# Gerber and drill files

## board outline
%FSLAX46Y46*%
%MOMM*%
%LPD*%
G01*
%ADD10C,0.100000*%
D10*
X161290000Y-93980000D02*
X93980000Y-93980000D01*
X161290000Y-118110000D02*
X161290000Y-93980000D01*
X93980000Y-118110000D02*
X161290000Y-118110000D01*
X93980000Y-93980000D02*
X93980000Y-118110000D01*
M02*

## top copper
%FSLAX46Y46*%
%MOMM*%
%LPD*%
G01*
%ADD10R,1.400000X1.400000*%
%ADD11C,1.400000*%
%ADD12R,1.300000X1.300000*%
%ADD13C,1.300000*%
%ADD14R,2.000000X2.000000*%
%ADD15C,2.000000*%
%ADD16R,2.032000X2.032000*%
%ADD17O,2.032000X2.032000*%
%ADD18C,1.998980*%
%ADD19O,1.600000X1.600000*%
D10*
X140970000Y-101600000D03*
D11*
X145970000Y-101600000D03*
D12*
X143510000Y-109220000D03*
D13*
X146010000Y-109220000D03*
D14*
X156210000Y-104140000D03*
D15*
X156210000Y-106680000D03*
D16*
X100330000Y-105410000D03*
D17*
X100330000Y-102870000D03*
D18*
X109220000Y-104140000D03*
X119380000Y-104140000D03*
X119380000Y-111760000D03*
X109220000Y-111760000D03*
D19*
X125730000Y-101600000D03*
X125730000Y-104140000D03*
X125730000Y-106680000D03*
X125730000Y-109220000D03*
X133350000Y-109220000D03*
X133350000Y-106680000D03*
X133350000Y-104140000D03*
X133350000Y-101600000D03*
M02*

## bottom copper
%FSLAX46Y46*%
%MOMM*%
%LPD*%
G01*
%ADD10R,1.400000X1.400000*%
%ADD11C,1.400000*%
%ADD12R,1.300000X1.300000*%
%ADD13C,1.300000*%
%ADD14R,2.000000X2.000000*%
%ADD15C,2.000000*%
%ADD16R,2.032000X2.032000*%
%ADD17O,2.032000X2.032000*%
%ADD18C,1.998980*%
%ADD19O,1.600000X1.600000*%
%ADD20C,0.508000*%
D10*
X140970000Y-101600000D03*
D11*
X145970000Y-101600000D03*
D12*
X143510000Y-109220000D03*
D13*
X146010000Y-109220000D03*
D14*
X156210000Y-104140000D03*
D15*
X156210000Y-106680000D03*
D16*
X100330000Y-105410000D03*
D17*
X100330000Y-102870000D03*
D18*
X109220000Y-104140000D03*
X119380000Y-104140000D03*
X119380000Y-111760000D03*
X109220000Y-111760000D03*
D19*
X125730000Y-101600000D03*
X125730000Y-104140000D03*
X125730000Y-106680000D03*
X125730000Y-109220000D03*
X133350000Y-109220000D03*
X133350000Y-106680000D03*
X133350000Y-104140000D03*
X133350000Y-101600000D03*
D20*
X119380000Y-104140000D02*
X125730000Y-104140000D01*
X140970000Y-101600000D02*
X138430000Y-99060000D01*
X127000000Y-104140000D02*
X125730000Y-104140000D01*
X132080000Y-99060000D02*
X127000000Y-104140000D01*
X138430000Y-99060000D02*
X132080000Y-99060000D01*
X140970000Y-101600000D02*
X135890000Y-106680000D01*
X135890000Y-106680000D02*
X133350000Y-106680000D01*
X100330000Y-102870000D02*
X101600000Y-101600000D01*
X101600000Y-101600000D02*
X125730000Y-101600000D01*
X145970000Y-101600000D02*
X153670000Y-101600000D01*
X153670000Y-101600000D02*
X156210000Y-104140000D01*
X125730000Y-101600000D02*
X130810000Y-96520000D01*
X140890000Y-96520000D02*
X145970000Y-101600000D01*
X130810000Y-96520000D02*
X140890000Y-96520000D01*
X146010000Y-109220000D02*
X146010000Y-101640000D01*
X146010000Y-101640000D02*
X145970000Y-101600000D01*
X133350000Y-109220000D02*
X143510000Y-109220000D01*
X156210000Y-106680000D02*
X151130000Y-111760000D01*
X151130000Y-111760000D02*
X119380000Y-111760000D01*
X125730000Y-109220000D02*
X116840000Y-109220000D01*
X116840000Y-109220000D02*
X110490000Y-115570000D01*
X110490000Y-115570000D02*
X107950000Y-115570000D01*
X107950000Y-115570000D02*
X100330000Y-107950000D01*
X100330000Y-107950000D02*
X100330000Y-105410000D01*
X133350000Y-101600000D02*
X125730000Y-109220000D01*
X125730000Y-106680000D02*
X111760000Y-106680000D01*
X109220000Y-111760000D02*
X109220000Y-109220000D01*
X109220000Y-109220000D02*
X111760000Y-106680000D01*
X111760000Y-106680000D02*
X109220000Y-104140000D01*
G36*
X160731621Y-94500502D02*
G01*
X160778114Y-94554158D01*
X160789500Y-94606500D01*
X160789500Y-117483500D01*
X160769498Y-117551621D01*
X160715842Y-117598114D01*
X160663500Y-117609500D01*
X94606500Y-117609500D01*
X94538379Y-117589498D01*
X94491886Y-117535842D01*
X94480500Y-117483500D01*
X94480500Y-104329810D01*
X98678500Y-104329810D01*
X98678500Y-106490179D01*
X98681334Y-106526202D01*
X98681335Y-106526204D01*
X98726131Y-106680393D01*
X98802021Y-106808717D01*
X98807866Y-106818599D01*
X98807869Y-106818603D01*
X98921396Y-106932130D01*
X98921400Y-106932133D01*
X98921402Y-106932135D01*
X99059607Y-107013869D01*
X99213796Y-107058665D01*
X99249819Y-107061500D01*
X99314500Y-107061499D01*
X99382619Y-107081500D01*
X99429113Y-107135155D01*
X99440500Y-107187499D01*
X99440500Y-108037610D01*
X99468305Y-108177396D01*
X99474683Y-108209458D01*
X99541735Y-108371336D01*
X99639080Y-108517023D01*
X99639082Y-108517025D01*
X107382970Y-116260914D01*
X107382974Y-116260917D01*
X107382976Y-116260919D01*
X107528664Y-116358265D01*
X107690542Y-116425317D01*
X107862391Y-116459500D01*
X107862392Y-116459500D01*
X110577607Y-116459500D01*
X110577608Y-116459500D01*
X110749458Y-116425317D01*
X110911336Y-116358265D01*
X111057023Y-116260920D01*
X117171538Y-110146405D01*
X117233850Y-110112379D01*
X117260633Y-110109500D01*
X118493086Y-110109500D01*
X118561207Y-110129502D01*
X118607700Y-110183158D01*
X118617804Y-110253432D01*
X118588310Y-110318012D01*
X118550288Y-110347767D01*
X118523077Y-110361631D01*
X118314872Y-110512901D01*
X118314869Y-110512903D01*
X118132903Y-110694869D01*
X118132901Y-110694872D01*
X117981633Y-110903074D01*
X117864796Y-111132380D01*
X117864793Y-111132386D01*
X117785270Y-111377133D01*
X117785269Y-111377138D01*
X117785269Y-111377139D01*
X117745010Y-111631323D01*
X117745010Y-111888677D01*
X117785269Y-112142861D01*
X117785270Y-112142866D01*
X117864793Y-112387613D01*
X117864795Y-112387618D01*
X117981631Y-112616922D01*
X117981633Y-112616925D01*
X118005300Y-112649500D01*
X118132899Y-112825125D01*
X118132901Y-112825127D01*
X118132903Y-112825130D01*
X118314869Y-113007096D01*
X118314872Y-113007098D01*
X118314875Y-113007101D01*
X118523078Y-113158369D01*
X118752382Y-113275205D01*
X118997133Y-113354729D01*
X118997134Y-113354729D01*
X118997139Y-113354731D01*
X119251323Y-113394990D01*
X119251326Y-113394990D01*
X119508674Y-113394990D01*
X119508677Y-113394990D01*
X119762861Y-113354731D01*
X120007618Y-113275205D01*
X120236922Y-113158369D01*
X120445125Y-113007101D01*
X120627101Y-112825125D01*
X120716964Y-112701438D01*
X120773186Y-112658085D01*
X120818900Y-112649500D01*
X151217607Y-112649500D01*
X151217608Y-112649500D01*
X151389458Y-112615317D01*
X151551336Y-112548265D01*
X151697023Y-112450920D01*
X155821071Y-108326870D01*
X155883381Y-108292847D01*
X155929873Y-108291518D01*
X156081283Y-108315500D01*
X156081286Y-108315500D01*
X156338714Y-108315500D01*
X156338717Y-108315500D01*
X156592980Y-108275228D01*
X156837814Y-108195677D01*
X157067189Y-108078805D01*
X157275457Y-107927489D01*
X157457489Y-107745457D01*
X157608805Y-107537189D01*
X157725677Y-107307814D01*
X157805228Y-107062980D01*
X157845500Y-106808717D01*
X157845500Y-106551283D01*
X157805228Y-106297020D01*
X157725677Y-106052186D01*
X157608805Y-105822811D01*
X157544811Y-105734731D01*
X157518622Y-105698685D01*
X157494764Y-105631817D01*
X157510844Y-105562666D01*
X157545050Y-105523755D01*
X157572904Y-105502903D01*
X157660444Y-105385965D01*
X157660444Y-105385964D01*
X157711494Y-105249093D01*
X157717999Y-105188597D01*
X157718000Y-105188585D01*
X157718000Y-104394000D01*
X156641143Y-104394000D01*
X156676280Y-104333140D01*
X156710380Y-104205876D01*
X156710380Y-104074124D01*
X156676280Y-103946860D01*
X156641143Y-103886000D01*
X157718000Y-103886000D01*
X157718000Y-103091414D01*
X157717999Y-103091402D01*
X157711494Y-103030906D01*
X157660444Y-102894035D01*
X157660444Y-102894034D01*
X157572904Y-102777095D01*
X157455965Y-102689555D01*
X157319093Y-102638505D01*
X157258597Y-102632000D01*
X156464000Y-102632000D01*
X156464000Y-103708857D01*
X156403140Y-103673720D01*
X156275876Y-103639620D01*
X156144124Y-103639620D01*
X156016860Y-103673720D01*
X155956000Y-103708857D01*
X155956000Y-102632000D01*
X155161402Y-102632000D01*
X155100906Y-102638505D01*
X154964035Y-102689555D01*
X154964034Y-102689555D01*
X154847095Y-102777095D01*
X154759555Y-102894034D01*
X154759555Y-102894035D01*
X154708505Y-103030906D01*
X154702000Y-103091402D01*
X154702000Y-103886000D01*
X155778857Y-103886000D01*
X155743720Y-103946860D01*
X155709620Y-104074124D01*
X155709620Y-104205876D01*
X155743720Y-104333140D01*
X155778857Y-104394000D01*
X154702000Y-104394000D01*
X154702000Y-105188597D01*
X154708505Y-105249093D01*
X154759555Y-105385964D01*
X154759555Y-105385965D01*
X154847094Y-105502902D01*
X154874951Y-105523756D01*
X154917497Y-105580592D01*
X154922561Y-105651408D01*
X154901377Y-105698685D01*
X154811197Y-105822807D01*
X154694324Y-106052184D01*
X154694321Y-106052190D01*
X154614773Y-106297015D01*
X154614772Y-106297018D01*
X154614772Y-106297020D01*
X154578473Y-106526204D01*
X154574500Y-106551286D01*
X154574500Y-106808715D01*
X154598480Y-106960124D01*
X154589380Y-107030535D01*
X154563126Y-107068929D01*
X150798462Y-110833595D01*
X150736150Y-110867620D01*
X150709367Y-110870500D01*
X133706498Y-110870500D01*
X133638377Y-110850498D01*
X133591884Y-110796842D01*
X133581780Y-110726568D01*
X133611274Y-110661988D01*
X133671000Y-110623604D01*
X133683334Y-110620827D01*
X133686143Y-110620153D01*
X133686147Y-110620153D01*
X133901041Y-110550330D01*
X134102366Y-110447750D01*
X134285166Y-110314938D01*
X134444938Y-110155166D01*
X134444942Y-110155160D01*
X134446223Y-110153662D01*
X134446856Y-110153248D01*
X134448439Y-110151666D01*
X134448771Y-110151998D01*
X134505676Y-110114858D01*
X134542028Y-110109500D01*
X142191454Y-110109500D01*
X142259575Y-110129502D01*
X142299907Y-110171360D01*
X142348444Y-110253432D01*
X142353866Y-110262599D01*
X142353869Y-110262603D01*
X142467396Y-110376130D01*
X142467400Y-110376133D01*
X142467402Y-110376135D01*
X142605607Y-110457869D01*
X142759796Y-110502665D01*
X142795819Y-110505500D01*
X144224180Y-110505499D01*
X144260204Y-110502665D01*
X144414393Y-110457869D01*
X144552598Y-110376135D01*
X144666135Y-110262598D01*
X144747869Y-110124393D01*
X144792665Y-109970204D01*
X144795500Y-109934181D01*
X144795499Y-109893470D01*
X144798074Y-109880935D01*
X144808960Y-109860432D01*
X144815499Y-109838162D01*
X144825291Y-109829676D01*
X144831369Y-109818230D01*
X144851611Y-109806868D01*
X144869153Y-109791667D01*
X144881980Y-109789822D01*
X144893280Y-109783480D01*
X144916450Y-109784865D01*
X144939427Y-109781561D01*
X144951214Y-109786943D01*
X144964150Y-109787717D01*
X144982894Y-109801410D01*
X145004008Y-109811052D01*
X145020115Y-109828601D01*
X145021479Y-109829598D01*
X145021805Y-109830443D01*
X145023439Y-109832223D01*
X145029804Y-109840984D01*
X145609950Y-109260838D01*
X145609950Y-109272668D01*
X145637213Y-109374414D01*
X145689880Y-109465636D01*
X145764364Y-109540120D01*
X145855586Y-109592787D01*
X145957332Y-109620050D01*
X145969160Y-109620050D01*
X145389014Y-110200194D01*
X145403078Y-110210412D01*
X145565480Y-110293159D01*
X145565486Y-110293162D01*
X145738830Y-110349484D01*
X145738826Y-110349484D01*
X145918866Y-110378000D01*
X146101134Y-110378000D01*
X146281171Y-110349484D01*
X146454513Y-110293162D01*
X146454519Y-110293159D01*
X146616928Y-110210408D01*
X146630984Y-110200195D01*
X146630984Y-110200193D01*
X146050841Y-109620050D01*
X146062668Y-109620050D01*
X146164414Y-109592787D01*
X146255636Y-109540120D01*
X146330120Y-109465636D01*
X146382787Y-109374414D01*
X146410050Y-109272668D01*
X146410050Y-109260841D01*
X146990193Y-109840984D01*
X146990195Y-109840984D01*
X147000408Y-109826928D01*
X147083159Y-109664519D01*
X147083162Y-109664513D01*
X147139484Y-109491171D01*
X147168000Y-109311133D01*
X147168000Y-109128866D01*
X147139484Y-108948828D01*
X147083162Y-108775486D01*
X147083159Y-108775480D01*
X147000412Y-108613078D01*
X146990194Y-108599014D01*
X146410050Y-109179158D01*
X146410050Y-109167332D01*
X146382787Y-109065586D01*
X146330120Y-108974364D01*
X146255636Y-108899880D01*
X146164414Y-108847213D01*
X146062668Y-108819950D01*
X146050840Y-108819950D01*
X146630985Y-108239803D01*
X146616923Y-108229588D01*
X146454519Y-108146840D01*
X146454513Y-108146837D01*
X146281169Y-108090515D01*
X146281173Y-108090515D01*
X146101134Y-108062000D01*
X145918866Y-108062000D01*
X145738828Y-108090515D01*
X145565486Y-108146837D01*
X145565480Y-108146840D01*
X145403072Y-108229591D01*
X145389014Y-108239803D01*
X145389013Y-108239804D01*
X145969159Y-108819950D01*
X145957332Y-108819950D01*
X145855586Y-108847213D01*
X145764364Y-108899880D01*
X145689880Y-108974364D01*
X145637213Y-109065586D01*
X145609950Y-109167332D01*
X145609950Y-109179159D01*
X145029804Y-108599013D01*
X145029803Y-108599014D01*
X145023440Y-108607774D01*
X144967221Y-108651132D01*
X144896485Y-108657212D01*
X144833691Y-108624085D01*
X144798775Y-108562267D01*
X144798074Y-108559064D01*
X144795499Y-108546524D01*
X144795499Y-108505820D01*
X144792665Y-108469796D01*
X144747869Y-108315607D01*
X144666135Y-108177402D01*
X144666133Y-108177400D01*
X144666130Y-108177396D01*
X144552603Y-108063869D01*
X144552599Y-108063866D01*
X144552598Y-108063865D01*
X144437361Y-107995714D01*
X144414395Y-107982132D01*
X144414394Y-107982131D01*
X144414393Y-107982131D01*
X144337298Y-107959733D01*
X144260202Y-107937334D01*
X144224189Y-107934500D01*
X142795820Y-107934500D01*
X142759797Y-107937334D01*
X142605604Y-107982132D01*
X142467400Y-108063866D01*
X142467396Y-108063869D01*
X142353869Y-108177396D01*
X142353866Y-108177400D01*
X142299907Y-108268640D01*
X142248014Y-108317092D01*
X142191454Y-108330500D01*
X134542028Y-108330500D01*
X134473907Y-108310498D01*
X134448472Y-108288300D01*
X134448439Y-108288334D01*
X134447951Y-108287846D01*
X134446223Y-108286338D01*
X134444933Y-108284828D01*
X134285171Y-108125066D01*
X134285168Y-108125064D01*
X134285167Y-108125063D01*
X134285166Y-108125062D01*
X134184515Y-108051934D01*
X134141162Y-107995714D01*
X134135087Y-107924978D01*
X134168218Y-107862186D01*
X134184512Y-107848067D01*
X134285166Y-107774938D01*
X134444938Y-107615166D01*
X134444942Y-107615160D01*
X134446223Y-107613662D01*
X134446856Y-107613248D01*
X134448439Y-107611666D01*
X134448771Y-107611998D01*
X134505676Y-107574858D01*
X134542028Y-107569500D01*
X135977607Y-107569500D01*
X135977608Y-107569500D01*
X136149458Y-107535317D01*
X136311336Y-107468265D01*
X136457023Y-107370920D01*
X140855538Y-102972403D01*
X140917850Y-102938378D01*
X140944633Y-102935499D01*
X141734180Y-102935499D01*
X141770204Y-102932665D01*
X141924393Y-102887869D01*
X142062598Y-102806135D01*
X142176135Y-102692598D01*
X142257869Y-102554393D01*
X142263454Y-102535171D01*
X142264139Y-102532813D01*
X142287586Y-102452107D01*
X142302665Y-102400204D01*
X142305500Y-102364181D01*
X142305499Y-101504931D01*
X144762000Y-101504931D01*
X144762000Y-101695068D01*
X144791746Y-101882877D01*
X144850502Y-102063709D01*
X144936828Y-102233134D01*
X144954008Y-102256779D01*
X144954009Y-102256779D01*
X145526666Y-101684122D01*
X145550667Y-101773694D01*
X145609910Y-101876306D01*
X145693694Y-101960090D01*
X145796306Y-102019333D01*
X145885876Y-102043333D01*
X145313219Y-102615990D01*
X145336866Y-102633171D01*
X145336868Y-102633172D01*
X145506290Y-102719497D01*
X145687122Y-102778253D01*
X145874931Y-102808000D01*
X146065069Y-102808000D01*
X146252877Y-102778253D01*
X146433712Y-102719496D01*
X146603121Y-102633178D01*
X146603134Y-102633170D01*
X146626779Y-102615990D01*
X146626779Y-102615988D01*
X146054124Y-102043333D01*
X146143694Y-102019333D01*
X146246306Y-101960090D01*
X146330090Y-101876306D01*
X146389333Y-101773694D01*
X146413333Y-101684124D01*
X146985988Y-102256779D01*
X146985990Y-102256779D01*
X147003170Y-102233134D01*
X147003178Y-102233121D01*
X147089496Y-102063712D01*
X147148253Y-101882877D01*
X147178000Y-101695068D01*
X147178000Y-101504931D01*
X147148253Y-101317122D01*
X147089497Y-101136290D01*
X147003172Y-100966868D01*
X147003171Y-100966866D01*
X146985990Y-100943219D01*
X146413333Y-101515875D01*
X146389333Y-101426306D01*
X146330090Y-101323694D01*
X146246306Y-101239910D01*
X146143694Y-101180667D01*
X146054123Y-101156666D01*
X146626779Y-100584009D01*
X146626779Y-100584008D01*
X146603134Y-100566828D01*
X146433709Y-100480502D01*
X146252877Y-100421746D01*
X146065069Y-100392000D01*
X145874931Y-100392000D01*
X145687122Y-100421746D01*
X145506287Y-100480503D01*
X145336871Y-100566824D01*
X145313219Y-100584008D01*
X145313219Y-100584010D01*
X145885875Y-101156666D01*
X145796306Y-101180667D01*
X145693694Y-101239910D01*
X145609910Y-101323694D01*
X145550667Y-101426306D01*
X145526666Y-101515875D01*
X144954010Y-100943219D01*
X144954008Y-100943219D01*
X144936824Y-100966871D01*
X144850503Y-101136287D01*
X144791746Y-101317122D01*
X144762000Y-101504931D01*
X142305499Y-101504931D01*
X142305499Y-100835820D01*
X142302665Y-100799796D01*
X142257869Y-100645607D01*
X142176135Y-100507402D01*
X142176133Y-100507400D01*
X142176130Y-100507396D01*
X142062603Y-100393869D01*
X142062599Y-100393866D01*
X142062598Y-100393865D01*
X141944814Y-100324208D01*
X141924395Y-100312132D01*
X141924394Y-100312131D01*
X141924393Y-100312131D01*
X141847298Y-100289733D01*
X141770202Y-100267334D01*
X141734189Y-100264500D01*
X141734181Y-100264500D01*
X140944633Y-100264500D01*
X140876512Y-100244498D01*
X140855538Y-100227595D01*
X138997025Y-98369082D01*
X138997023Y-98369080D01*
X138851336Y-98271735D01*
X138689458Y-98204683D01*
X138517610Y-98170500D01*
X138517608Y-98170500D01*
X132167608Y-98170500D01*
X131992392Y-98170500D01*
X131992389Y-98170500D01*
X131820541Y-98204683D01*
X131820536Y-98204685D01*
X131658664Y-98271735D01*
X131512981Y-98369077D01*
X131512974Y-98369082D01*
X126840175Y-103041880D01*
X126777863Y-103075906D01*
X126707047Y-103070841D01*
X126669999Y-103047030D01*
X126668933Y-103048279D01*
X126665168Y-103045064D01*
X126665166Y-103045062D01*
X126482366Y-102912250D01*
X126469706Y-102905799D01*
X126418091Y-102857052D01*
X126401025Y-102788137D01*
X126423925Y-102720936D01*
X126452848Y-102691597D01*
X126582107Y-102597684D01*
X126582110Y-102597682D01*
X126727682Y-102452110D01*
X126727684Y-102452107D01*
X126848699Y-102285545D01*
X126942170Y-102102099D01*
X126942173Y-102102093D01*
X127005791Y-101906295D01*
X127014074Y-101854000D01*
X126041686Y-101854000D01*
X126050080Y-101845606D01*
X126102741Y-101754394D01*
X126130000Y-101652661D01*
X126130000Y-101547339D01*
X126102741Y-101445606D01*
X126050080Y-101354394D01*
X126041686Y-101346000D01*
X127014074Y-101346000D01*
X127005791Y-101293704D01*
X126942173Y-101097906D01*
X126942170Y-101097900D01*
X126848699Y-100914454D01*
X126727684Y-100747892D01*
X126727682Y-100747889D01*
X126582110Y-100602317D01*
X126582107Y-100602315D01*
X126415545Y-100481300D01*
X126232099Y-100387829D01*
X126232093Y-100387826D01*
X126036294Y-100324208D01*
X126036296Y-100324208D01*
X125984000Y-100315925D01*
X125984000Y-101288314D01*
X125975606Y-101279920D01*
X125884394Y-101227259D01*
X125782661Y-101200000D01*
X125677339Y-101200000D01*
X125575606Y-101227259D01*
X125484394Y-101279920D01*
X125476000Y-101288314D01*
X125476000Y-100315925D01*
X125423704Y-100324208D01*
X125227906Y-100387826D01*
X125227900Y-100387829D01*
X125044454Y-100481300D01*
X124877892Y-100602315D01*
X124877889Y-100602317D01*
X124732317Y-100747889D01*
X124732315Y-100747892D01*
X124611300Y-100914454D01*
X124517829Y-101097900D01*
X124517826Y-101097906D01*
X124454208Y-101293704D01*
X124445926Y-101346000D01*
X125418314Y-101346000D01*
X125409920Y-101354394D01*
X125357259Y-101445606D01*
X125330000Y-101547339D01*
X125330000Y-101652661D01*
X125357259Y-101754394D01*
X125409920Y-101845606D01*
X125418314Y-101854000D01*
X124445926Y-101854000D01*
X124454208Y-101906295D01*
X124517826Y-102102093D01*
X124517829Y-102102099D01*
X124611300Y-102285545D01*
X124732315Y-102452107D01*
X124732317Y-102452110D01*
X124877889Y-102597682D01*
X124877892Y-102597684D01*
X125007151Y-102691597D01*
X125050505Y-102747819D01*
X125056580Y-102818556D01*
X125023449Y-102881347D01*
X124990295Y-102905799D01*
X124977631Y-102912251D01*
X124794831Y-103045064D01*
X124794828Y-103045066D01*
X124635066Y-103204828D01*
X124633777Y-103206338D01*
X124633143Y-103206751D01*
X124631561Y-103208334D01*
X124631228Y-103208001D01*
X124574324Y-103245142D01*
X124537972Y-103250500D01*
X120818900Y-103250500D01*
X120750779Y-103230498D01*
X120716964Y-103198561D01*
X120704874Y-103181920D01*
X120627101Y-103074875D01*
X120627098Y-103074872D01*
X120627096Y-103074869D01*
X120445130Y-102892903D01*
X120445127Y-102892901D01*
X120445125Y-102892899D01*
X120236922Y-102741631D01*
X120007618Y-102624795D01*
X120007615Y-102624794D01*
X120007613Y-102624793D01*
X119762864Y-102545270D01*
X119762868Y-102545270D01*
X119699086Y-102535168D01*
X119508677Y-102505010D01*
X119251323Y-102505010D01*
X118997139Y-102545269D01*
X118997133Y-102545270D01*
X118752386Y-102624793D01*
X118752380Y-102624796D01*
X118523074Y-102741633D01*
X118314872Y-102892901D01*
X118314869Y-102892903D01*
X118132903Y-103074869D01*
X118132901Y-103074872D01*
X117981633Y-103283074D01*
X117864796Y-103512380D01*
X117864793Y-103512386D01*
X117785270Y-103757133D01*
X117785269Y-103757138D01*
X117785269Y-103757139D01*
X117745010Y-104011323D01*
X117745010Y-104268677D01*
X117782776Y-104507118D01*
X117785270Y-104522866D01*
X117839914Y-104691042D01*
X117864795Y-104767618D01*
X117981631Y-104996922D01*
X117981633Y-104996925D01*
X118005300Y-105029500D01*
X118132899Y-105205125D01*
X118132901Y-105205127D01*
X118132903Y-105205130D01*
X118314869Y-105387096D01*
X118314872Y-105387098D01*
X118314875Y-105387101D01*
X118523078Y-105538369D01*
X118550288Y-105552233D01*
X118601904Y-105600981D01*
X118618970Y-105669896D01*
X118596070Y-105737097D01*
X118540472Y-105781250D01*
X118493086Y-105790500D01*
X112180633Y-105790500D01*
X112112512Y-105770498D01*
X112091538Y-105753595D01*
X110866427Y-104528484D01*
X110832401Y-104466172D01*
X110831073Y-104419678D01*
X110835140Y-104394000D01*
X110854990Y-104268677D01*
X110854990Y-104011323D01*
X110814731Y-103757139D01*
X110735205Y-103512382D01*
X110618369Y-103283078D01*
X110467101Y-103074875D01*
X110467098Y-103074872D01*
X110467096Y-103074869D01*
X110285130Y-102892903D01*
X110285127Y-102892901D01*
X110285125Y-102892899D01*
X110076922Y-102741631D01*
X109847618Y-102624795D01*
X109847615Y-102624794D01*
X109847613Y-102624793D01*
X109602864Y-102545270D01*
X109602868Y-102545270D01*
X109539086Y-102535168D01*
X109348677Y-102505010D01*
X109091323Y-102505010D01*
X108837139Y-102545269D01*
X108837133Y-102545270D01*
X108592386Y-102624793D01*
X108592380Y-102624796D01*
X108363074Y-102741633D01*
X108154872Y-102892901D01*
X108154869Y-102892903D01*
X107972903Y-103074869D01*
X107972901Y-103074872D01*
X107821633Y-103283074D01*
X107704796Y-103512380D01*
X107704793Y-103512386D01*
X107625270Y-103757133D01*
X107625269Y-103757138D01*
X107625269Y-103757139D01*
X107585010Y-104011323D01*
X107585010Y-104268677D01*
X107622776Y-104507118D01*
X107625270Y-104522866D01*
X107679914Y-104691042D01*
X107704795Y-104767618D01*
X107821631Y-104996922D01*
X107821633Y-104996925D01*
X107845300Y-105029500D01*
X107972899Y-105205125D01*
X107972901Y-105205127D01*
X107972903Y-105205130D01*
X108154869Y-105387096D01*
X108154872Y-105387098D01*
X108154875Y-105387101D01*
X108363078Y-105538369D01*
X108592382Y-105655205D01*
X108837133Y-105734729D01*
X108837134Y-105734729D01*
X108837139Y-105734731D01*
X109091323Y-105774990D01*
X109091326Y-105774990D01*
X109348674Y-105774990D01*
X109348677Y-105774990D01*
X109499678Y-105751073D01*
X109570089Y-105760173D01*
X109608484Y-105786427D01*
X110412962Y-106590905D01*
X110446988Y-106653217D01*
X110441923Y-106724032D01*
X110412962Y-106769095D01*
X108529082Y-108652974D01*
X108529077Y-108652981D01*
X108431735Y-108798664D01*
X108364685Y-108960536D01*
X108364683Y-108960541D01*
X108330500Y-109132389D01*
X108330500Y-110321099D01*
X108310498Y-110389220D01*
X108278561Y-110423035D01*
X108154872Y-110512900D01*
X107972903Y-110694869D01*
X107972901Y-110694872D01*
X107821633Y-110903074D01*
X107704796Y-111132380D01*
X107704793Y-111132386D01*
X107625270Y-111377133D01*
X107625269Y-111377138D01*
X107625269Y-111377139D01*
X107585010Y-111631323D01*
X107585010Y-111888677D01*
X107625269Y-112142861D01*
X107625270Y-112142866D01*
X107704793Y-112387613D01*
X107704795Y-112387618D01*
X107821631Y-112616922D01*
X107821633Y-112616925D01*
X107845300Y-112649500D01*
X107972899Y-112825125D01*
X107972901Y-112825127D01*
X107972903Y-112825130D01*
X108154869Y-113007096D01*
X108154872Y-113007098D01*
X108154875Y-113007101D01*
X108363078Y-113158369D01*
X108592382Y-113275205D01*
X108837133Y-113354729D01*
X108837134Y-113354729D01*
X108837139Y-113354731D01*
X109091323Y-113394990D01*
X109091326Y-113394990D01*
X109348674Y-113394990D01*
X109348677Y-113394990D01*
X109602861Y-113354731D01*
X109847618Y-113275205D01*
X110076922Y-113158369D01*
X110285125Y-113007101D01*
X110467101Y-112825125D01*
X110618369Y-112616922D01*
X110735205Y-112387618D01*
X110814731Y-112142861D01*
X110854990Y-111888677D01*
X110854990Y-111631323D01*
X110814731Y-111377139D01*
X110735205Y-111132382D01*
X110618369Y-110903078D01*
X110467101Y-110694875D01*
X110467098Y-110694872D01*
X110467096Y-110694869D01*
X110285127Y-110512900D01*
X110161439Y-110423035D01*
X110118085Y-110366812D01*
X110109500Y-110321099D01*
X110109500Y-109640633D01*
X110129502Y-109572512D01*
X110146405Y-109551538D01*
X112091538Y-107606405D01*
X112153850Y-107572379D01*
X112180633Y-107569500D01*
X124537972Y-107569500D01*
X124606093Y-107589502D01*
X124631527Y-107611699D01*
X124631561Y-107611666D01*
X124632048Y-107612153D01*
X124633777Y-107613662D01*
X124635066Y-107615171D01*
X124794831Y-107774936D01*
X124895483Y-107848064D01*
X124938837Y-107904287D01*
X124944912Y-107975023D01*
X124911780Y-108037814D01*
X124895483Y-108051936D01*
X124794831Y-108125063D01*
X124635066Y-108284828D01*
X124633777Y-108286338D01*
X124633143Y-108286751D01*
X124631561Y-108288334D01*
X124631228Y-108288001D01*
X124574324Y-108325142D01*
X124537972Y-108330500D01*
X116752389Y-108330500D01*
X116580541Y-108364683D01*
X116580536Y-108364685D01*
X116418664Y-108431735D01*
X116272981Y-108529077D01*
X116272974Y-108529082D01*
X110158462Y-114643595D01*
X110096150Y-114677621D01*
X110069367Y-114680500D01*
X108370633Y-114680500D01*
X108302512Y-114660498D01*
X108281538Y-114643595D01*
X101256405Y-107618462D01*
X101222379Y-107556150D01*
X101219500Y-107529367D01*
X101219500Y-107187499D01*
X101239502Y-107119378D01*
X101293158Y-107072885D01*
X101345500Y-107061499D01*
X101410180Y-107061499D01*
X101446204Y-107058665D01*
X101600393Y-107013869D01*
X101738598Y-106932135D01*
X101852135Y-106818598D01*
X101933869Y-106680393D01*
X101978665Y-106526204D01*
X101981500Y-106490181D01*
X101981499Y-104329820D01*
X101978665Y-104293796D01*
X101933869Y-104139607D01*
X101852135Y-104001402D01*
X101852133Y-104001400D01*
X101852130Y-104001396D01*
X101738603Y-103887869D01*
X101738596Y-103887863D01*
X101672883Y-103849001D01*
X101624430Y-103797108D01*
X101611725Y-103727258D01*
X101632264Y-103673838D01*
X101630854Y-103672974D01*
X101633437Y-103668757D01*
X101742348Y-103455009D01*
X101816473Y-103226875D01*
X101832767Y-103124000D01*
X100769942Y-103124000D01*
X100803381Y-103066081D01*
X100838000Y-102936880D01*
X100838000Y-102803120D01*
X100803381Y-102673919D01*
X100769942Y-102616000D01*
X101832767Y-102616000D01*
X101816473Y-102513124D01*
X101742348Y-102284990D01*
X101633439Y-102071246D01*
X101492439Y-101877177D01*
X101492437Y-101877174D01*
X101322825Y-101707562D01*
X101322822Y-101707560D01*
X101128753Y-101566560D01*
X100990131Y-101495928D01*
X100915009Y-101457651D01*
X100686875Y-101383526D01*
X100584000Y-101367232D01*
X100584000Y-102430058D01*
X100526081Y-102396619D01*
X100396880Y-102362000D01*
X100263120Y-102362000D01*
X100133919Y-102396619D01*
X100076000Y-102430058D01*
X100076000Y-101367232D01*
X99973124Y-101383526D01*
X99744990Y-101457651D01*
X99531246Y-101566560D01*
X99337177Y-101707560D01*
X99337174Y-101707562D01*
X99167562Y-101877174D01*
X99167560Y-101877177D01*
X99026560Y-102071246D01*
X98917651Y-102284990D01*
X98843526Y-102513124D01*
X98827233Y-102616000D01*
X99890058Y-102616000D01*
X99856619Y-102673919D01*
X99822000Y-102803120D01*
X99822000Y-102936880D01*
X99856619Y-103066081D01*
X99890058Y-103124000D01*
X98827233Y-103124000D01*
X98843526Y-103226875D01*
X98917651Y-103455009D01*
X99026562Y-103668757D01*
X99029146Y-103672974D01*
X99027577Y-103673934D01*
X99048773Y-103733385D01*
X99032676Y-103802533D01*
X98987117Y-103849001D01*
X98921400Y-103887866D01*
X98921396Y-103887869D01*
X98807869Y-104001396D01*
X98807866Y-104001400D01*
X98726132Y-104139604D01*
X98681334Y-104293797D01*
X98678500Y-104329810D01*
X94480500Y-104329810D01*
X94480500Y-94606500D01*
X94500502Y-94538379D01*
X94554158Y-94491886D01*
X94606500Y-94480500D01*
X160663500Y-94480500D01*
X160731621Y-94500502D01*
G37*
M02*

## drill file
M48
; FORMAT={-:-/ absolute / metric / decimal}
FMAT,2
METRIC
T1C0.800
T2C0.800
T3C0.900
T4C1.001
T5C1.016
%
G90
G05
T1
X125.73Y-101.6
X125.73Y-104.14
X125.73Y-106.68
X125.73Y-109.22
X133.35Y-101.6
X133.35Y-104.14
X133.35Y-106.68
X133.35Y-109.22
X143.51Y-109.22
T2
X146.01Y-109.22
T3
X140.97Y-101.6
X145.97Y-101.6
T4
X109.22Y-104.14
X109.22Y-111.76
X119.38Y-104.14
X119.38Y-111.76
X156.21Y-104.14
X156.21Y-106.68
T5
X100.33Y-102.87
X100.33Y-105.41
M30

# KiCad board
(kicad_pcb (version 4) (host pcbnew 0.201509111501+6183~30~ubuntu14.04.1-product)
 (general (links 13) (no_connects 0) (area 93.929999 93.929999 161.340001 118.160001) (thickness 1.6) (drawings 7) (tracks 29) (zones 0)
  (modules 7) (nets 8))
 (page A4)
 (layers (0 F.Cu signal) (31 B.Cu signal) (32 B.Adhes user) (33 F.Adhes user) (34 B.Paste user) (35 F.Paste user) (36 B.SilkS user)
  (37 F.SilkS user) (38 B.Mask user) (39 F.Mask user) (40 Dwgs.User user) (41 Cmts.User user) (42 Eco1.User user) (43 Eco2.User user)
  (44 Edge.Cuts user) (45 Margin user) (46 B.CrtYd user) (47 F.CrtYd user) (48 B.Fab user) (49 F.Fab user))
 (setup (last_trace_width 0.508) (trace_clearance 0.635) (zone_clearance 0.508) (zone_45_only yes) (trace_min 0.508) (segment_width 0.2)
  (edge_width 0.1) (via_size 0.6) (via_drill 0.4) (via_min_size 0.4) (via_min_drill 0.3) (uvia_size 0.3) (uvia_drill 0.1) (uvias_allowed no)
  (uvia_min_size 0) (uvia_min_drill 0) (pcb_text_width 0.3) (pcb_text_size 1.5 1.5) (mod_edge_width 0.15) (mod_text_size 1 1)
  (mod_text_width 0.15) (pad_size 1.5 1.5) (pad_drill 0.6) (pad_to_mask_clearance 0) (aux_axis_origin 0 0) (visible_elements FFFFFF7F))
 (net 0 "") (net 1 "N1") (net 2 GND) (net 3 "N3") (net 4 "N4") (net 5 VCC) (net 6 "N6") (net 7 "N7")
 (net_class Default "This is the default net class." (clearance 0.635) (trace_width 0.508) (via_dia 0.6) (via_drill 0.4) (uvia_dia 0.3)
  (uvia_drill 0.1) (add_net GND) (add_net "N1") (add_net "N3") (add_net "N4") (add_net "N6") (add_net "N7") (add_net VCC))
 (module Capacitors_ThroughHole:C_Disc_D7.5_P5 (layer F.Cu) (at 140.97 101.6)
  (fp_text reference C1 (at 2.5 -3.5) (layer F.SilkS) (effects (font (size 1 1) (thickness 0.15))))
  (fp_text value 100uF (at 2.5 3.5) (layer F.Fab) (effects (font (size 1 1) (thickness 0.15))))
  (pad 1 thru_hole rect (at 0 0) (size 1.4 1.4) (drill 0.9) (layers *.Cu *.Mask F.SilkS) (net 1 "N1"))
  (pad 2 thru_hole circle (at 5 0) (size 1.4 1.4) (drill 0.9) (layers *.Cu *.Mask F.SilkS) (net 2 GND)))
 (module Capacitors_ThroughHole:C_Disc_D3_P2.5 (layer F.Cu) (at 143.51 109.22)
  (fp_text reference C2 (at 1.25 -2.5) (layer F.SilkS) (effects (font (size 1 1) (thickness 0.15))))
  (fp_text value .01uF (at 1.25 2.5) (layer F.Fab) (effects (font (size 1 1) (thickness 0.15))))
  (pad 1 thru_hole rect (at 0 0) (size 1.3 1.3) (drill 0.8) (layers *.Cu *.Mask F.SilkS) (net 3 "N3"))
  (pad 2 thru_hole circle (at 2.5 0) (size 1.3 1.3) (drill 0.8001) (layers *.Cu *.Mask F.SilkS) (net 2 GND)))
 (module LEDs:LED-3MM (layer F.Cu) (at 156.21 104.14 270)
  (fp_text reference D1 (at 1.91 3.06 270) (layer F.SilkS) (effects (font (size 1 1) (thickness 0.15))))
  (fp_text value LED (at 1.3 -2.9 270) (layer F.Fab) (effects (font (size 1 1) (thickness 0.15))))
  (pad 1 thru_hole rect (at 0 0) (size 2 2) (drill 1.00076) (layers *.Cu *.Mask F.SilkS) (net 2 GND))
  (pad 2 thru_hole circle (at 2.54 0 270) (size 2 2) (drill 1.00076) (layers *.Cu *.Mask F.SilkS) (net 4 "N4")))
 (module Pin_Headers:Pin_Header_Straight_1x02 (layer F.Cu) (at 100.33 105.41 180)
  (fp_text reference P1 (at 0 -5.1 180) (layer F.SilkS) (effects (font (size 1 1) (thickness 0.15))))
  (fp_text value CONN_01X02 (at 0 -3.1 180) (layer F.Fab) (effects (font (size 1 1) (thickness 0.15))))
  (pad 1 thru_hole rect (at 0 0 180) (size 2.032 2.032) (drill 1.016) (layers *.Cu *.Mask F.SilkS) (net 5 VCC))
  (pad 2 thru_hole oval (at 0 2.54 180) (size 2.032 2.032) (drill 1.016) (layers *.Cu *.Mask F.SilkS) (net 2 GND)))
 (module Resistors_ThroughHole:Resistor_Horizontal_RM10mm (layer F.Cu) (at 114.3 104.14)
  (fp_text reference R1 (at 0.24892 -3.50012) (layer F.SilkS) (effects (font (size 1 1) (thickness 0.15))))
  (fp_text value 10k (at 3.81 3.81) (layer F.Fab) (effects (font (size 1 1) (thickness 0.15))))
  (pad 1 thru_hole circle (at -5.08 0) (size 1.99898 1.99898) (drill 1.00076) (layers *.Cu *.SilkS *.Mask) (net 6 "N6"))
  (pad 2 thru_hole circle (at 5.08 0) (size 1.99898 1.99898) (drill 1.00076) (layers *.Cu *.SilkS *.Mask) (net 1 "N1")))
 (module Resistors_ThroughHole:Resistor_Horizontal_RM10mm (layer F.Cu) (at 114.3 111.76 180)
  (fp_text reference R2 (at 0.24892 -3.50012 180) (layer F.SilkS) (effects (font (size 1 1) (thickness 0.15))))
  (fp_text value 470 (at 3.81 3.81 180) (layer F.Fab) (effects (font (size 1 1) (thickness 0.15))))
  (pad 1 thru_hole circle (at -5.08 0 180) (size 1.99898 1.99898) (drill 1.00076) (layers *.Cu *.SilkS *.Mask) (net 4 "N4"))
  (pad 2 thru_hole circle (at 5.08 0 180) (size 1.99898 1.99898) (drill 1.00076) (layers *.Cu *.SilkS *.Mask) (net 6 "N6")))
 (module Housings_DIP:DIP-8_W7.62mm (layer F.Cu) (at 125.73 101.6)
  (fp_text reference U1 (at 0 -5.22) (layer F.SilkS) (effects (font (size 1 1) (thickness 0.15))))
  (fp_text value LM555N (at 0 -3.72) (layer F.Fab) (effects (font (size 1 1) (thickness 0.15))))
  (pad 1 thru_hole oval (at 0 0) (size 1.6 1.6) (drill 0.8) (layers *.Cu *.Mask F.SilkS) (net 2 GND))
  (pad 2 thru_hole oval (at 0 2.54) (size 1.6 1.6) (drill 0.8) (layers *.Cu *.Mask F.SilkS) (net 1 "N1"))
  (pad 3 thru_hole oval (at 0 5.08) (size 1.6 1.6) (drill 0.8) (layers *.Cu *.Mask F.SilkS) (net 6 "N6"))
  (pad 4 thru_hole oval (at 0 7.62) (size 1.6 1.6) (drill 0.8) (layers *.Cu *.Mask F.SilkS) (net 5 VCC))
  (pad 5 thru_hole oval (at 7.62 7.62) (size 1.6 1.6) (drill 0.8) (layers *.Cu *.Mask F.SilkS) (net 3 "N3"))
  (pad 6 thru_hole oval (at 7.62 5.08) (size 1.6 1.6) (drill 0.8) (layers *.Cu *.Mask F.SilkS) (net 1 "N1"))
  (pad 7 thru_hole oval (at 7.62 2.54) (size 1.6 1.6) (drill 0.8) (layers *.Cu *.Mask F.SilkS) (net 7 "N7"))
  (pad 8 thru_hole oval (at 7.62 0) (size 1.6 1.6) (drill 0.8) (layers *.Cu *.Mask F.SilkS) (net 5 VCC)))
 (gr_line (start 161.29 93.98) (end 93.98 93.98) (angle 90) (layer Edge.Cuts) (width 0.1))
 (gr_line (start 161.29 118.11) (end 161.29 93.98) (angle 90) (layer Edge.Cuts) (width 0.1))
 (gr_line (start 93.98 118.11) (end 161.29 118.11) (angle 90) (layer Edge.Cuts) (width 0.1))
 (gr_line (start 93.98 93.98) (end 93.98 118.11) (angle 90) (layer Edge.Cuts) (width 0.1))
 (segment (start 119.38 104.14) (end 125.73 104.14) (width 0.508) (layer B.Cu) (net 1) (status 20))
 (segment (start 140.97 101.6) (end 138.43 99.06) (width 0.508) (layer B.Cu) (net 1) (status 10))
 (segment (start 127 104.14) (end 125.73 104.14) (width 0.508) (layer B.Cu) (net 1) (status 20))
 (segment (start 132.08 99.06) (end 127 104.14) (width 0.508) (layer B.Cu) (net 1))
 (segment (start 138.43 99.06) (end 132.08 99.06) (width 0.508) (layer B.Cu) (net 1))
 (segment (start 140.97 101.6) (end 135.89 106.68) (width 0.508) (layer B.Cu) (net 1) (status 10))
 (segment (start 135.89 106.68) (end 133.35 106.68) (width 0.508) (layer B.Cu) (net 1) (status 20))
 (segment (start 100.33 102.87) (end 101.6 101.6) (width 0.508) (layer B.Cu) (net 2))
 (segment (start 101.6 101.6) (end 125.73 101.6) (width 0.508) (layer B.Cu) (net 2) (status 20))
 (segment (start 145.97 101.6) (end 153.67 101.6) (width 0.508) (layer B.Cu) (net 2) (status 10))
 (segment (start 153.67 101.6) (end 156.21 104.14) (width 0.508) (layer B.Cu) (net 2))
 (segment (start 125.73 101.6) (end 130.81 96.52) (width 0.508) (layer B.Cu) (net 2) (status 10))
 (segment (start 140.89 96.52) (end 145.97 101.6) (width 0.508) (layer B.Cu) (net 2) (status 20))
 (segment (start 130.81 96.52) (end 140.89 96.52) (width 0.508) (layer B.Cu) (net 2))
 (segment (start 146.01 109.22) (end 146.01 101.64) (width 0.508) (layer B.Cu) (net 2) (status 20))
 (segment (start 146.01 101.64) (end 145.97 101.6) (width 0.508) (layer B.Cu) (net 2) (status 30))
 (segment (start 133.35 109.22) (end 143.51 109.22) (width 0.508) (layer B.Cu) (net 3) (status 10))
 (segment (start 156.21 106.68) (end 151.13 111.76) (width 0.508) (layer B.Cu) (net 4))
 (segment (start 151.13 111.76) (end 119.38 111.76) (width 0.508) (layer B.Cu) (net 4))
 (segment (start 125.73 109.22) (end 116.84 109.22) (width 0.508) (layer B.Cu) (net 5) (status 10))
 (segment (start 116.84 109.22) (end 110.49 115.57) (width 0.508) (layer B.Cu) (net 5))
 (segment (start 110.49 115.57) (end 107.95 115.57) (width 0.508) (layer B.Cu) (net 5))
 (segment (start 107.95 115.57) (end 100.33 107.95) (width 0.508) (layer B.Cu) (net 5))
 (segment (start 100.33 107.95) (end 100.33 105.41) (width 0.508) (layer B.Cu) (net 5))
 (segment (start 133.35 101.6) (end 125.73 109.22) (width 0.508) (layer B.Cu) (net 5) (status 30))
 (segment (start 125.73 106.68) (end 111.76 106.68) (width 0.508) (layer B.Cu) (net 6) (status 10))
 (segment (start 109.22 111.76) (end 109.22 109.22) (width 0.508) (layer B.Cu) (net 6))
 (segment (start 109.22 109.22) (end 111.76 106.68) (width 0.508) (layer B.Cu) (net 6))
 (segment (start 111.76 106.68) (end 109.22 104.14) (width 0.508) (layer B.Cu) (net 6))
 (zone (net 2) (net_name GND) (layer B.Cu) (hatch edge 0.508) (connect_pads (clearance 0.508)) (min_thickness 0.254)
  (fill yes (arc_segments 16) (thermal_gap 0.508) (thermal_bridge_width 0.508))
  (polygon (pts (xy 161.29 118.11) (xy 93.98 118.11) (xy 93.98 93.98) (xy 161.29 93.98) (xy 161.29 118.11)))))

